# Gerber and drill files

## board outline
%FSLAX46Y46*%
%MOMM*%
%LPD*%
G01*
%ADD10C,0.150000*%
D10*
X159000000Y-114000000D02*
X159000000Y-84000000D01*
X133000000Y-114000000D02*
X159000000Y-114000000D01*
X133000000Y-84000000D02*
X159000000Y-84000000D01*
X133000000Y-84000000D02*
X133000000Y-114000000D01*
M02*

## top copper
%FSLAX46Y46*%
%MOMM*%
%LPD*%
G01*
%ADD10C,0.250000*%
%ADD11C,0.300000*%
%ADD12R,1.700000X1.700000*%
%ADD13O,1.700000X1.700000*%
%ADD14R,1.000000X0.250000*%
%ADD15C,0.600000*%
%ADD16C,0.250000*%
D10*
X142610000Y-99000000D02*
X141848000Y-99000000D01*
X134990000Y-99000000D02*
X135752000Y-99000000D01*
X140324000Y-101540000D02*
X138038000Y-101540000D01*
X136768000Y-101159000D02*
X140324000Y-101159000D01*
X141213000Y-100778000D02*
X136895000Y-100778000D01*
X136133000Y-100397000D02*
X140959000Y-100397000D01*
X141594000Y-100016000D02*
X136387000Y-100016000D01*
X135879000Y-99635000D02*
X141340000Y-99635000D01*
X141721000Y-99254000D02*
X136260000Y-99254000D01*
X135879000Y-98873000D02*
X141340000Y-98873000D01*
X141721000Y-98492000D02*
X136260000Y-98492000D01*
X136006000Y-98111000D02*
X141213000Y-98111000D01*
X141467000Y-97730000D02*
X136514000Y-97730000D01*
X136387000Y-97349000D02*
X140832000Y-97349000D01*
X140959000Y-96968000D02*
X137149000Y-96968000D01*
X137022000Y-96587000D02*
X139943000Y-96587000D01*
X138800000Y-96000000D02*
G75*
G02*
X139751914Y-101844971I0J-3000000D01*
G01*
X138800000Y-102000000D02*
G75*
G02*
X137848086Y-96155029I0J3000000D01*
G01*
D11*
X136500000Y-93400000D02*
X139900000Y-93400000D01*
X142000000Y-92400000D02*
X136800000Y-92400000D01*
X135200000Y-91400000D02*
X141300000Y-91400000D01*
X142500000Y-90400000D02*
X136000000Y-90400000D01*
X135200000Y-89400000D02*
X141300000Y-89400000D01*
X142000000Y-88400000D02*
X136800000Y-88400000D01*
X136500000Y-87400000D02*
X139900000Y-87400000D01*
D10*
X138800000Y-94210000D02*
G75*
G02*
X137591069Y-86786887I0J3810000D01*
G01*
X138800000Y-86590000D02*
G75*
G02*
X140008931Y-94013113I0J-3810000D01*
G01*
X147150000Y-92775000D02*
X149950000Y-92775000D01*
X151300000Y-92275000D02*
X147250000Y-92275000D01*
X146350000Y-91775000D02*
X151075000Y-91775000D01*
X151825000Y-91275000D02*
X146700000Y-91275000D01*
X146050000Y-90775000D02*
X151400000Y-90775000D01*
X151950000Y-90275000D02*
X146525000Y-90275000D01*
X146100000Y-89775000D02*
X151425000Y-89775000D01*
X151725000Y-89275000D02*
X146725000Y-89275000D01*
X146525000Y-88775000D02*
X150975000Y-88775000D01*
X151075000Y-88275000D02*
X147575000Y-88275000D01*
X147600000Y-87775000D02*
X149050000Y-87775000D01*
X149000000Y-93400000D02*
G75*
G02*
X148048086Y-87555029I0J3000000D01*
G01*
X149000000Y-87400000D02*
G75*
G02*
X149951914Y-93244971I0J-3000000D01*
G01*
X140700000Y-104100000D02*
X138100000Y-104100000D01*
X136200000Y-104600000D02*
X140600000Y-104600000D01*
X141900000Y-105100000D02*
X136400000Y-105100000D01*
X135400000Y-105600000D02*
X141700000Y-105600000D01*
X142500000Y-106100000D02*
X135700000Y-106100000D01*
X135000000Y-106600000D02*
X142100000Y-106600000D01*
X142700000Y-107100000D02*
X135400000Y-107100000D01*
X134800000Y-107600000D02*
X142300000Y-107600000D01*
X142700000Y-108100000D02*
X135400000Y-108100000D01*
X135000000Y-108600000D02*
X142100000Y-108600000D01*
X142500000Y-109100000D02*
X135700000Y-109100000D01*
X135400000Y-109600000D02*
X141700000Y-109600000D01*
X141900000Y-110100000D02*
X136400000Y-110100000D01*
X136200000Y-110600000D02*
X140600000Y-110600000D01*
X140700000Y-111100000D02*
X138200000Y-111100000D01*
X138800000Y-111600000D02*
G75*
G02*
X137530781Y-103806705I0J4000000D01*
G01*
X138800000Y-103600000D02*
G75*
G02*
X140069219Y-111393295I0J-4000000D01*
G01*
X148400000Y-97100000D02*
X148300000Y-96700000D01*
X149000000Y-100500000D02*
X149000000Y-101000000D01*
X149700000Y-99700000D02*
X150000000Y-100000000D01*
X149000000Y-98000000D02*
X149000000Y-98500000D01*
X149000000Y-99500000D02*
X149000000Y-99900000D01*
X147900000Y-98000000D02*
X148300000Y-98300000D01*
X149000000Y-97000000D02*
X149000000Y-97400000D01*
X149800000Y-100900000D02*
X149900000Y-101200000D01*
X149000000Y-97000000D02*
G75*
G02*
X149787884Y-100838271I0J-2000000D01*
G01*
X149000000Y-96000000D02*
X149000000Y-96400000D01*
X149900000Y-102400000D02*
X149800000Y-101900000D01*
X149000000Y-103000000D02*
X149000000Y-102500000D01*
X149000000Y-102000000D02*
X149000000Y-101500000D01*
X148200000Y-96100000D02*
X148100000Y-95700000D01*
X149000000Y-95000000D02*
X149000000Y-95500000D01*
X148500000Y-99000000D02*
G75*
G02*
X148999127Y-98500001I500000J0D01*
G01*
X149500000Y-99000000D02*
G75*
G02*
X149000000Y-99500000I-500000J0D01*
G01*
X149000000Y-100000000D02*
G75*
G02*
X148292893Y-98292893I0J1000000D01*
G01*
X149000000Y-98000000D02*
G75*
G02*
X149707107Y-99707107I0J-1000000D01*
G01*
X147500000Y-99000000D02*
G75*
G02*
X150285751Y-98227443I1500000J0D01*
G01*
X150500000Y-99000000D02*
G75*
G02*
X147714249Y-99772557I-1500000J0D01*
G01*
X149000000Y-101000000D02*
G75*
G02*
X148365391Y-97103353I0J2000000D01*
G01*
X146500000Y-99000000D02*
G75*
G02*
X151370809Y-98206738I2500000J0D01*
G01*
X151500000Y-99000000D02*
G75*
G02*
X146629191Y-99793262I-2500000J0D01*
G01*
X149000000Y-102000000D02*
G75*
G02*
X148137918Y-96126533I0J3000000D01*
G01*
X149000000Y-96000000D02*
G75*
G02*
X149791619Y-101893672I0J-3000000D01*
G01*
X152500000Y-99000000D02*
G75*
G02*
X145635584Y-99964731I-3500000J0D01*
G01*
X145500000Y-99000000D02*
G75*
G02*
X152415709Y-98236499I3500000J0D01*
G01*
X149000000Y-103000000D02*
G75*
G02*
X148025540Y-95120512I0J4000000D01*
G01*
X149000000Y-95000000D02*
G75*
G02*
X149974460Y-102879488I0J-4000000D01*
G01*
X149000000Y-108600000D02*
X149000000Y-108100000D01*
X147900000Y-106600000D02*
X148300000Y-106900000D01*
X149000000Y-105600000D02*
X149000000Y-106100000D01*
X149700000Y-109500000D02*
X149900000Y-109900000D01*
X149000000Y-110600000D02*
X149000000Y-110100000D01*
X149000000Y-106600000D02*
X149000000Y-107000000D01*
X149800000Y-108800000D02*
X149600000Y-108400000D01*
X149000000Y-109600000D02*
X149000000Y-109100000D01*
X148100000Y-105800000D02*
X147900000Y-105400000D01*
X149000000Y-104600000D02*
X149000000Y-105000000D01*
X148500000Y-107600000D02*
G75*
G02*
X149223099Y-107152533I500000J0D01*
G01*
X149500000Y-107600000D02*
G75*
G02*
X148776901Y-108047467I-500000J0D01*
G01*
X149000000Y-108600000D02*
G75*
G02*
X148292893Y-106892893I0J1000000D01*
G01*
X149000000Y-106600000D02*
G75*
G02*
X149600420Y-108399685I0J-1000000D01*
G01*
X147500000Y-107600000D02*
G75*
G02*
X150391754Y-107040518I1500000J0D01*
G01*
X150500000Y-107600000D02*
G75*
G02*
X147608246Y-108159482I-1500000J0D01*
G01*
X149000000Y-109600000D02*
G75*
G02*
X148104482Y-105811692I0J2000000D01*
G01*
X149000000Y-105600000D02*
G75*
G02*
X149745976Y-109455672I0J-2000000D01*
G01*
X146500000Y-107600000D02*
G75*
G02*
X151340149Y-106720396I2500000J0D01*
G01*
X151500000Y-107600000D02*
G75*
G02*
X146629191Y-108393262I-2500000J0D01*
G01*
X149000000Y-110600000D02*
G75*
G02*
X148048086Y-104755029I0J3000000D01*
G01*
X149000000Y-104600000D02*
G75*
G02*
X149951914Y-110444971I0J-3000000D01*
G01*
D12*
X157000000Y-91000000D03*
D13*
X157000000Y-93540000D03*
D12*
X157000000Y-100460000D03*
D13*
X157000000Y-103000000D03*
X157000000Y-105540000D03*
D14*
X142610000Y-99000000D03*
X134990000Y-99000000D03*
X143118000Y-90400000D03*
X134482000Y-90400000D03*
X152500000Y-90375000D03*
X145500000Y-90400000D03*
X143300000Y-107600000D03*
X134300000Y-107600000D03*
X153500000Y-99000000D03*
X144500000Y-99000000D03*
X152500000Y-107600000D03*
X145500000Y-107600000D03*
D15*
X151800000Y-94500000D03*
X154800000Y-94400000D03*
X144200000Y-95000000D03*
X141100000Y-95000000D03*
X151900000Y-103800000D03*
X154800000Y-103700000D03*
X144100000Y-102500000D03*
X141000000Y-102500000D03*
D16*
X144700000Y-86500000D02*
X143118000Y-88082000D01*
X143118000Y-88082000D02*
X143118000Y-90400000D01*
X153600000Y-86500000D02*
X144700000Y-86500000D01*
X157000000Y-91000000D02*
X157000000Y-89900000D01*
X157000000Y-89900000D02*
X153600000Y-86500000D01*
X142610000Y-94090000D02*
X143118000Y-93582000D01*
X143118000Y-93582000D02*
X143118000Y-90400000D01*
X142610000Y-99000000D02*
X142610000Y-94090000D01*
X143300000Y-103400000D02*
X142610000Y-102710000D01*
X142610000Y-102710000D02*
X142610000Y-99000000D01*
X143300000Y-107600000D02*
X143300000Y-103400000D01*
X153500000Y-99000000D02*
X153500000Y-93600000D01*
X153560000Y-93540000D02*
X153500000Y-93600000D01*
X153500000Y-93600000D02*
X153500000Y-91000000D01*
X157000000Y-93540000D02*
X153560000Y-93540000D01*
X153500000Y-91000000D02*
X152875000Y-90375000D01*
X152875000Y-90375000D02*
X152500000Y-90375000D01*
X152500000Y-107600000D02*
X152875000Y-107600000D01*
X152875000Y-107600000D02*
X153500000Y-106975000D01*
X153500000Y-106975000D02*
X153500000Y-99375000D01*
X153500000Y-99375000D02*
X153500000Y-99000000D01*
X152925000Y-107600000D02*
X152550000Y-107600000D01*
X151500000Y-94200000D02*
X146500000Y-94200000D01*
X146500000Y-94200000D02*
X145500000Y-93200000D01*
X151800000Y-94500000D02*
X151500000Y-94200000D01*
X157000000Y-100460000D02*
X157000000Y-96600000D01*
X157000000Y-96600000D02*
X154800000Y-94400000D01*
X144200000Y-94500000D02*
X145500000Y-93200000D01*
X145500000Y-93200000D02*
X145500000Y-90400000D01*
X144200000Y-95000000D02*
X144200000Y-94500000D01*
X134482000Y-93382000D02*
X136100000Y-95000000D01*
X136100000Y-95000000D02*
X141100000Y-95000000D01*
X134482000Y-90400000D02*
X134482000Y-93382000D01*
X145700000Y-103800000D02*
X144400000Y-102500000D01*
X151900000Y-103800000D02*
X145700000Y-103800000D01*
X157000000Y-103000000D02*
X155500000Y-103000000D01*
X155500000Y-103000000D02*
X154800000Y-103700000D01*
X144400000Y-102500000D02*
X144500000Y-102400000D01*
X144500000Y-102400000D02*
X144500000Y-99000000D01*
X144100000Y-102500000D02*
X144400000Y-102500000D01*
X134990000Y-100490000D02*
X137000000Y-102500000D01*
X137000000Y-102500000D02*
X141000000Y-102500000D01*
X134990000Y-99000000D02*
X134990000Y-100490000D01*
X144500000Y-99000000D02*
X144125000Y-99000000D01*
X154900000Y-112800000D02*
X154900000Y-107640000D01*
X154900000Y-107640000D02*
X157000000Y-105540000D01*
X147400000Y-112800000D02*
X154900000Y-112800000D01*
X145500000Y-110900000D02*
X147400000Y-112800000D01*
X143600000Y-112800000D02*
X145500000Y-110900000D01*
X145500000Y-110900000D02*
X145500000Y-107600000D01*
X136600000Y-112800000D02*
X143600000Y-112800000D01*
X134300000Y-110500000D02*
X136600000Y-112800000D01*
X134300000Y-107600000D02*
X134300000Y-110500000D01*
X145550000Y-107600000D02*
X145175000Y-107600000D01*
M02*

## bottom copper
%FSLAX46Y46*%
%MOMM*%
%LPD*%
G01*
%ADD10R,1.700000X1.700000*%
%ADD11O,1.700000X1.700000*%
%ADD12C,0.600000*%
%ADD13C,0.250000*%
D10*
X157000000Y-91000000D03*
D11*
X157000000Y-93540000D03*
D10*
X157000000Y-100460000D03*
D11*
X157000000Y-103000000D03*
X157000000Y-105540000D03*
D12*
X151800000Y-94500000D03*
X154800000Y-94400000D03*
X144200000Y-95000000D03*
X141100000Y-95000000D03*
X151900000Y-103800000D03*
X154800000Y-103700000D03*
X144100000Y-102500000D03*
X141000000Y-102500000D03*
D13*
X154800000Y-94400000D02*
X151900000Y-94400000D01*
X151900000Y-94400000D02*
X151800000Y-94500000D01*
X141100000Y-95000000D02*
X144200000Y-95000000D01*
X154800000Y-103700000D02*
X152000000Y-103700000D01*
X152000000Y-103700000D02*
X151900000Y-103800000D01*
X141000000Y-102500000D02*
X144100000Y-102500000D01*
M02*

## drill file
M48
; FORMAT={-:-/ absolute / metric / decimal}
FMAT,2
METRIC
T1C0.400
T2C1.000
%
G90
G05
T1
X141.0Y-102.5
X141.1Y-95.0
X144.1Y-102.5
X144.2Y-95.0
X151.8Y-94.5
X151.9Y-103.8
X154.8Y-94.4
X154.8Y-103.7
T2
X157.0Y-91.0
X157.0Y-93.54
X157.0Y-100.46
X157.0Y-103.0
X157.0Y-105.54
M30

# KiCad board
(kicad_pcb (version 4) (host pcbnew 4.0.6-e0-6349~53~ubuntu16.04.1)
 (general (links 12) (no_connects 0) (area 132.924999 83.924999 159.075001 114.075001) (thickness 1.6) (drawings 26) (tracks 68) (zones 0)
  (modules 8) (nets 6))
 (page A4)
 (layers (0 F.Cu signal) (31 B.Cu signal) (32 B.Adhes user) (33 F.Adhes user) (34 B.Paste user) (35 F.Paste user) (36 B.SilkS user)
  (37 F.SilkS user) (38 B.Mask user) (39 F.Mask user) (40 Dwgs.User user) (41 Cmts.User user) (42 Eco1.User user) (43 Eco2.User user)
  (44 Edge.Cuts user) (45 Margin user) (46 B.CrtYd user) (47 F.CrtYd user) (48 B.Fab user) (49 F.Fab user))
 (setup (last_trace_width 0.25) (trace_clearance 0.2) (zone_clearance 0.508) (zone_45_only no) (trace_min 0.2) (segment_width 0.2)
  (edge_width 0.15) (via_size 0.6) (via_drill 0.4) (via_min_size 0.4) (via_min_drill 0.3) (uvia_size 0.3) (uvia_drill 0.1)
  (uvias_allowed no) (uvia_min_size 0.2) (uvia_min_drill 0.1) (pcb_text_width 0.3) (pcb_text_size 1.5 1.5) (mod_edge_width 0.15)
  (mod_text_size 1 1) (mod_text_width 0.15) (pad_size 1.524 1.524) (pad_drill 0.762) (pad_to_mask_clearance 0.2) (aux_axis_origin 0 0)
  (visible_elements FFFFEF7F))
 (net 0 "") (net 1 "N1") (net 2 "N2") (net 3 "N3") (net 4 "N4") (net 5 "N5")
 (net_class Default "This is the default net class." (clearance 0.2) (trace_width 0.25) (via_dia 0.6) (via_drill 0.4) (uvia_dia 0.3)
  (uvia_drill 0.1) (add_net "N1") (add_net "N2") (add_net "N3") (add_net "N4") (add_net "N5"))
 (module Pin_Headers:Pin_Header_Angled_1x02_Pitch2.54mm (layer F.Cu) (at 157 91)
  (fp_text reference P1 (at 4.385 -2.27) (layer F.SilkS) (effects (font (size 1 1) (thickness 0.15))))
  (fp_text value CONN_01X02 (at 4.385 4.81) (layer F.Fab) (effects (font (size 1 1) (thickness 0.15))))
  (pad 1 thru_hole rect (at 0 0) (size 1.7 1.7) (drill 1) (layers *.Cu *.Mask) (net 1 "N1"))
  (pad 2 thru_hole oval (at 0 2.54) (size 1.7 1.7) (drill 1) (layers *.Cu *.Mask) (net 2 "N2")))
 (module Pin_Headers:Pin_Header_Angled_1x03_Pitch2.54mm (layer F.Cu) (at 157 100.46)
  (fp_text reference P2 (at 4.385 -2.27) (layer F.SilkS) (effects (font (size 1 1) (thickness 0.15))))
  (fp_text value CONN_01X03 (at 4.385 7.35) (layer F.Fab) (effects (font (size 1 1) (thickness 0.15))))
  (pad 1 thru_hole rect (at 0 0) (size 1.7 1.7) (drill 1) (layers *.Cu *.Mask) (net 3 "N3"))
  (pad 2 thru_hole oval (at 0 2.54) (size 1.7 1.7) (drill 1) (layers *.Cu *.Mask) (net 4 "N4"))
  (pad 3 thru_hole oval (at 0 5.08) (size 1.7 1.7) (drill 1) (layers *.Cu *.Mask) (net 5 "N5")))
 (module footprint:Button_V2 (layer F.Cu) (at 138.8 99)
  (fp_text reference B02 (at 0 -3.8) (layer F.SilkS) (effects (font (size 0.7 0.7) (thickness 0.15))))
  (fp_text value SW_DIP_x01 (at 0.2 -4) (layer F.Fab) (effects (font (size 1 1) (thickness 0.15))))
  (fp_line (start 3.81 0) (end 3.048 0) (layer F.Cu) (width 0.25))
  (fp_line (start -3.81 0) (end -3.048 0) (layer F.Cu) (width 0.25))
  (fp_line (start 1.524 2.54) (end -0.762 2.54) (layer F.Cu) (width 0.25))
  (fp_line (start -2.032 2.159) (end 1.524 2.159) (layer F.Cu) (width 0.25))
  (fp_line (start 2.413 1.778) (end -1.905 1.778) (layer F.Cu) (width 0.25))
  (fp_line (start -2.667 1.397) (end 2.159 1.397) (layer F.Cu) (width 0.25))
  (fp_line (start 2.794 1.016) (end -2.413 1.016) (layer F.Cu) (width 0.25))
  (fp_line (start -2.921 0.635) (end 2.54 0.635) (layer F.Cu) (width 0.25))
  (fp_line (start 2.921 0.254) (end -2.54 0.254) (layer F.Cu) (width 0.25))
  (fp_line (start -2.921 -0.127) (end 2.54 -0.127) (layer F.Cu) (width 0.25))
  (fp_line (start 2.921 -0.508) (end -2.54 -0.508) (layer F.Cu) (width 0.25))
  (fp_line (start -2.794 -0.889) (end 2.413 -0.889) (layer F.Cu) (width 0.25))
  (fp_line (start 2.667 -1.27) (end -2.286 -1.27) (layer F.Cu) (width 0.25))
  (fp_line (start -2.413 -1.651) (end 2.032 -1.651) (layer F.Cu) (width 0.25))
  (fp_line (start 2.159 -2.032) (end -1.651 -2.032) (layer F.Cu) (width 0.25))
  (fp_line (start -1.778 -2.413) (end 1.143 -2.413) (layer F.Cu) (width 0.25))
  (fp_arc (start 0 0) (end 0 -3) (angle 161.5) (layer F.Cu) (width 0.25))
  (fp_arc (start 0 0) (end 0 3) (angle 161.5) (layer F.Cu) (width 0.25))
  (pad 1 smd rect (at 3.81 0) (size 1 0.25) (layers F.Cu F.Paste F.Mask) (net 1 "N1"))
  (pad 2 smd rect (at -3.81 0) (size 1 0.25) (layers F.Cu F.Paste F.Mask) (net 4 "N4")))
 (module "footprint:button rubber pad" (layer F.Cu) (at 138.8 90.4)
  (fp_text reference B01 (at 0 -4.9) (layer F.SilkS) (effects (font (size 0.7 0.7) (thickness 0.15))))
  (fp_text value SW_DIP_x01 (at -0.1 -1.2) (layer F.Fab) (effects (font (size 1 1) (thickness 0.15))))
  (fp_line (start -2.3 3) (end 1.1 3) (layer F.Cu) (width 0.3)) (fp_line (start 3.2 2) (end -2 2) (layer F.Cu) (width 0.3))
  (fp_line (start -3.6 1) (end 2.5 1) (layer F.Cu) (width 0.3))
  (fp_line (start 3.7 0) (end -2.8 0) (layer F.Cu) (width 0.3))
  (fp_line (start -3.6 -1) (end 2.5 -1) (layer F.Cu) (width 0.3))
  (fp_line (start 3.2 -2) (end -2 -2) (layer F.Cu) (width 0.3))
  (fp_line (start -2.3 -3) (end 1.1 -3) (layer F.Cu) (width 0.3))
  (fp_arc (start 0 0) (end 0 3.81) (angle 161.5) (layer F.Cu) (width 0.25))
  (fp_arc (start 0 0) (end 0 -3.81) (angle 161.5) (layer F.Cu) (width 0.25))
  (pad 1 smd rect (at 4.318 0) (size 1 0.25) (layers F.Cu F.Paste F.Mask) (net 1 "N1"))
  (pad 2 smd rect (at -4.318 0) (size 1 0.25) (layers F.Cu F.Paste F.Mask) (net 3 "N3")))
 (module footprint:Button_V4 (layer F.Cu) (at 149 90.4)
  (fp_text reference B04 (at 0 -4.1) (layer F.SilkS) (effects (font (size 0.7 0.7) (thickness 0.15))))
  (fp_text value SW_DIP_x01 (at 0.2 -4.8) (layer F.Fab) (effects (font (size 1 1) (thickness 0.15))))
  (fp_line (start -1.85 2.375) (end 0.95 2.375) (layer F.Cu) (width 0.25))
  (fp_line (start 2.3 1.875) (end -1.75 1.875) (layer F.Cu) (width 0.25))
  (fp_line (start -2.65 1.375) (end 2.075 1.375) (layer F.Cu) (width 0.25))
  (fp_line (start 2.825 0.875) (end -2.3 0.875) (layer F.Cu) (width 0.25))
  (fp_line (start -2.95 0.375) (end 2.4 0.375) (layer F.Cu) (width 0.25))
  (fp_line (start 2.95 -0.125) (end -2.475 -0.125) (layer F.Cu) (width 0.25))
  (fp_line (start -2.9 -0.625) (end 2.425 -0.625) (layer F.Cu) (width 0.25))
  (fp_line (start 2.725 -1.125) (end -2.275 -1.125) (layer F.Cu) (width 0.25))
  (fp_line (start -2.475 -1.625) (end 1.975 -1.625) (layer F.Cu) (width 0.25))
  (fp_line (start 2.075 -2.125) (end -1.425 -2.125) (layer F.Cu) (width 0.25))
  (fp_line (start -1.4 -2.625) (end 0.05 -2.625) (layer F.Cu) (width 0.25))
  (fp_arc (start 0 0) (end 0 3) (angle 161.5) (layer F.Cu) (width 0.25))
  (fp_arc (start 0 0) (end 0 -3) (angle 161.5) (layer F.Cu) (width 0.25))
  (pad 1 smd rect (at 3.5 -0.025) (size 1 0.25) (layers F.Cu F.Paste F.Mask) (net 2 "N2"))
  (pad 2 smd rect (at -3.5 0) (size 1 0.25) (layers F.Cu F.Paste F.Mask) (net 3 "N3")))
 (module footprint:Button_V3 (layer F.Cu) (at 138.8 107.6)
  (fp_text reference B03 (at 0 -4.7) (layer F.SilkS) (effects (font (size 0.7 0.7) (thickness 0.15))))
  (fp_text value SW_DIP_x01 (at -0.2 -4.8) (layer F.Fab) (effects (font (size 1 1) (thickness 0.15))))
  (fp_line (start 1.9 -3.5) (end -0.7 -3.5) (layer F.Cu) (width 0.25))
  (fp_line (start -2.6 -3) (end 1.8 -3) (layer F.Cu) (width 0.25))
  (fp_line (start 3.1 -2.5) (end -2.4 -2.5) (layer F.Cu) (width 0.25))
  (fp_line (start -3.4 -2) (end 2.9 -2) (layer F.Cu) (width 0.25))
  (fp_line (start 3.7 -1.5) (end -3.1 -1.5) (layer F.Cu) (width 0.25))
  (fp_line (start -3.8 -1) (end 3.3 -1) (layer F.Cu) (width 0.25))
  (fp_line (start 3.9 -0.5) (end -3.4 -0.5) (layer F.Cu) (width 0.25)) (fp_line (start -4 0) (end 3.5 0) (layer F.Cu) (width 0.25))
  (fp_line (start 3.9 0.5) (end -3.4 0.5) (layer F.Cu) (width 0.25))
  (fp_line (start -3.8 1) (end 3.3 1) (layer F.Cu) (width 0.25))
  (fp_line (start 3.7 1.5) (end -3.1 1.5) (layer F.Cu) (width 0.25))
  (fp_line (start -3.4 2) (end 2.9 2) (layer F.Cu) (width 0.25))
  (fp_line (start 3.1 2.5) (end -2.4 2.5) (layer F.Cu) (width 0.25))
  (fp_line (start -2.6 3) (end 1.8 3) (layer F.Cu) (width 0.25))
  (fp_line (start 1.9 3.5) (end -0.6 3.5) (layer F.Cu) (width 0.25))
  (fp_arc (start 0 0) (end 0 4) (angle 161.5) (layer F.Cu) (width 0.25))
  (fp_arc (start 0 0) (end 0 -4) (angle 161.5) (layer F.Cu) (width 0.25))
  (pad 1 smd rect (at 4.5 0) (size 1 0.25) (layers F.Cu F.Paste F.Mask) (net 1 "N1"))
  (pad 2 smd rect (at -4.5 0) (size 1 0.25) (layers F.Cu F.Paste F.Mask) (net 5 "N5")))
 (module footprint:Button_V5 (layer F.Cu) (at 149 99)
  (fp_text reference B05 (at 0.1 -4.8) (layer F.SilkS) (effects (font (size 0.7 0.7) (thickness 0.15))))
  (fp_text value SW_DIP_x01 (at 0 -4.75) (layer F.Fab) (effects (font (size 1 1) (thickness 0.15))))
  (fp_line (start -0.6 -1.9) (end -0.7 -2.3) (layer F.Cu) (width 0.25)) (fp_line (start 0 1.5) (end 0 2) (layer F.Cu) (width 0.25))
  (fp_line (start 0.7 0.7) (end 1 1) (layer F.Cu) (width 0.25))
  (fp_line (start 0 -1) (end 0 -0.5) (layer F.Cu) (width 0.25))
  (fp_line (start 0 0.5) (end 0 0.9) (layer F.Cu) (width 0.25))
  (fp_line (start -1.1 -1) (end -0.7 -0.7) (layer F.Cu) (width 0.25))
  (fp_line (start 0 -2) (end 0 -1.6) (layer F.Cu) (width 0.25))
  (fp_line (start 0.8 1.9) (end 0.9 2.2) (layer F.Cu) (width 0.25))
  (fp_arc (start 0 0) (end 0 -2) (angle 156.8) (layer F.Cu) (width 0.25))
  (fp_line (start 0 -3) (end 0 -2.6) (layer F.Cu) (width 0.25))
  (fp_line (start 0.9 3.4) (end 0.8 2.9) (layer F.Cu) (width 0.25)) (fp_line (start 0 4) (end 0 3.5) (layer F.Cu) (width 0.25))
  (fp_line (start 0 3) (end 0 2.5) (layer F.Cu) (width 0.25))
  (fp_line (start -0.8 -2.9) (end -0.9 -3.3) (layer F.Cu) (width 0.25))
  (fp_line (start 0 -4) (end 0 -3.5) (layer F.Cu) (width 0.25))
  (fp_arc (start 0 0) (end -0.5 0) (angle 89.9) (layer F.Cu) (width 0.25))
  (fp_arc (start 0 0) (end 0.5 0) (angle 90) (layer F.Cu) (width 0.25))
  (fp_arc (start 0 0) (end 0 1) (angle 135) (layer F.Cu) (width 0.25))
  (fp_arc (start 0 0) (end 0 -1) (angle 135) (layer F.Cu) (width 0.25))
  (fp_arc (start 0 0) (end -1.5 0) (angle 149) (layer F.Cu) (width 0.25))
  (fp_arc (start 0 0) (end 1.5 0) (angle 149) (layer F.Cu) (width 0.25))
  (fp_arc (start 0 0) (end 0 2) (angle 161.5) (layer F.Cu) (width 0.25))
  (fp_arc (start 0 0) (end -2.5 0) (angle 161.5) (layer F.Cu) (width 0.25))
  (fp_arc (start 0 0) (end 2.5 0) (angle 161.5) (layer F.Cu) (width 0.25))
  (fp_arc (start 0 0) (end 0 3) (angle 163.3) (layer F.Cu) (width 0.25))
  (fp_arc (start 0 0) (end 0 -3) (angle 164.7) (layer F.Cu) (width 0.25))
  (fp_arc (start 0 0) (end 3.5 0) (angle 164) (layer F.Cu) (width 0.25))
  (fp_arc (start 0 0) (end -3.5 0) (angle 167.4) (layer F.Cu) (width 0.25))
  (fp_arc (start 0 0) (end 0 4) (angle 165.9) (layer F.Cu) (width 0.25))
  (fp_arc (start 0 0) (end 0 -4) (angle 165.9) (layer F.Cu) (width 0.25))
  (pad 1 smd rect (at 4.5 0) (size 1 0.25) (layers F.Cu F.Paste F.Mask) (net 2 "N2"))
  (pad 2 smd rect (at -4.5 0) (size 1 0.25) (layers F.Cu F.Paste F.Mask) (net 4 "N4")))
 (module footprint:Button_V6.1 (layer F.Cu) (at 149 107.6)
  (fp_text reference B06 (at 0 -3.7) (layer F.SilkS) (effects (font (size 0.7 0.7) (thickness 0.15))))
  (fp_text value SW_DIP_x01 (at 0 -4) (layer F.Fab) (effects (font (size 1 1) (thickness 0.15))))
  (fp_line (start 0 1) (end 0 0.5) (layer F.Cu) (width 0.25))
  (fp_line (start -1.1 -1) (end -0.7 -0.7) (layer F.Cu) (width 0.25))
  (fp_line (start 0 -2) (end 0 -1.5) (layer F.Cu) (width 0.25))
  (fp_line (start 0.7 1.9) (end 0.9 2.3) (layer F.Cu) (width 0.25)) (fp_line (start 0 3) (end 0 2.5) (layer F.Cu) (width 0.25))
  (fp_line (start 0 -1) (end 0 -0.6) (layer F.Cu) (width 0.25))
  (fp_line (start 0.8 1.2) (end 0.6 0.8) (layer F.Cu) (width 0.25)) (fp_line (start 0 2) (end 0 1.5) (layer F.Cu) (width 0.25))
  (fp_line (start -0.9 -1.8) (end -1.1 -2.2) (layer F.Cu) (width 0.25))
  (fp_line (start 0 -3) (end 0 -2.6) (layer F.Cu) (width 0.25))
  (fp_arc (start 0 0) (end -0.5 0) (angle 116.5) (layer F.Cu) (width 0.25))
  (fp_arc (start 0 0) (end 0.5 0) (angle 116.5) (layer F.Cu) (width 0.25))
  (fp_arc (start 0 0) (end 0 1) (angle 135) (layer F.Cu) (width 0.25))
  (fp_arc (start 0 0) (end 0 -1) (angle 143.1) (layer F.Cu) (width 0.25))
  (fp_arc (start 0 0) (end -1.5 0) (angle 158.1) (layer F.Cu) (width 0.25))
  (fp_arc (start 0 0) (end 1.5 0) (angle 158.1) (layer F.Cu) (width 0.25))
  (fp_arc (start 0 0) (end 0 2) (angle 153.4) (layer F.Cu) (width 0.25))
  (fp_arc (start 0 0) (end 0 -2) (angle 158.1) (layer F.Cu) (width 0.25))
  (fp_arc (start 0 0) (end -2.5 0) (angle 159.4) (layer F.Cu) (width 0.25))
  (fp_arc (start 0 0) (end 2.5 0) (angle 161.5) (layer F.Cu) (width 0.25))
  (fp_arc (start 0 0) (end 0 3) (angle 161.5) (layer F.Cu) (width 0.25))
  (fp_arc (start 0 0) (end 0 -3) (angle 161.5) (layer F.Cu) (width 0.25))
  (pad 1 smd rect (at 3.5 0) (size 1 0.25) (layers F.Cu F.Paste F.Mask) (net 2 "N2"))
  (pad 2 smd rect (at -3.5 0) (size 1 0.25) (layers F.Cu F.Paste F.Mask) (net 5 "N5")))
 (gr_line (start 159 114) (end 159 84) (layer Edge.Cuts) (width 0.15))
 (gr_line (start 133 114) (end 159 114) (layer Edge.Cuts) (width 0.15))
 (gr_line (start 133 84) (end 159 84) (layer Edge.Cuts) (width 0.15))
 (gr_line (start 133 84) (end 133 114) (layer Edge.Cuts) (width 0.15))
 (segment (start 144.7 86.5) (end 143.118 88.082) (width 0.25) (layer F.Cu) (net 1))
 (segment (start 143.118 88.082) (end 143.118 90.4) (width 0.25) (layer F.Cu) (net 1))
 (segment (start 153.6 86.5) (end 144.7 86.5) (width 0.25) (layer F.Cu) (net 1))
 (segment (start 157 91) (end 157 89.9) (width 0.25) (layer F.Cu) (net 1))
 (segment (start 157 89.9) (end 153.6 86.5) (width 0.25) (layer F.Cu) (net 1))
 (segment (start 142.61 94.09) (end 143.118 93.582) (width 0.25) (layer F.Cu) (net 1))
 (segment (start 143.118 93.582) (end 143.118 90.4) (width 0.25) (layer F.Cu) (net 1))
 (segment (start 142.61 99) (end 142.61 94.09) (width 0.25) (layer F.Cu) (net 1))
 (segment (start 143.3 103.4) (end 142.61 102.71) (width 0.25) (layer F.Cu) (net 1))
 (segment (start 142.61 102.71) (end 142.61 99) (width 0.25) (layer F.Cu) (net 1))
 (segment (start 143.3 107.6) (end 143.3 103.4) (width 0.25) (layer F.Cu) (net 1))
 (segment (start 153.5 99) (end 153.5 93.6) (width 0.25) (layer F.Cu) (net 2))
 (segment (start 153.56 93.54) (end 153.5 93.6) (width 0.25) (layer F.Cu) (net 2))
 (segment (start 153.5 93.6) (end 153.5 91) (width 0.25) (layer F.Cu) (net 2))
 (segment (start 157 93.54) (end 153.56 93.54) (width 0.25) (layer F.Cu) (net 2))
 (segment (start 153.5 91) (end 152.875 90.375) (width 0.25) (layer F.Cu) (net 2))
 (segment (start 152.875 90.375) (end 152.5 90.375) (width 0.25) (layer F.Cu) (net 2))
 (segment (start 152.5 107.6) (end 152.875 107.6) (width 0.25) (layer F.Cu) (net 2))
 (segment (start 152.875 107.6) (end 153.5 106.975) (width 0.25) (layer F.Cu) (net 2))
 (segment (start 153.5 106.975) (end 153.5 99.375) (width 0.25) (layer F.Cu) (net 2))
 (segment (start 153.5 99.375) (end 153.5 99) (width 0.25) (layer F.Cu) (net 2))
 (segment (start 152.925 107.6) (end 152.55 107.6) (width 0.25) (layer F.Cu) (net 2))
 (segment (start 151.5 94.2) (end 146.5 94.2) (width 0.25) (layer F.Cu) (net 3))
 (segment (start 146.5 94.2) (end 145.5 93.2) (width 0.25) (layer F.Cu) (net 3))
 (segment (start 151.8 94.5) (end 151.5 94.2) (width 0.25) (layer F.Cu) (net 3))
 (segment (start 154.8 94.4) (end 151.9 94.4) (width 0.25) (layer B.Cu) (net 3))
 (segment (start 151.9 94.4) (end 151.8 94.5) (width 0.25) (layer B.Cu) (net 3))
 (via (at 151.8 94.5) (size 0.6) (drill 0.4) (layers F.Cu B.Cu) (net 3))
 (segment (start 157 100.46) (end 157 96.6) (width 0.25) (layer F.Cu) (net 3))
 (segment (start 157 96.6) (end 154.8 94.4) (width 0.25) (layer F.Cu) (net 3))
 (via (at 154.8 94.4) (size 0.6) (drill 0.4) (layers F.Cu B.Cu) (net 3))
 (segment (start 144.2 94.5) (end 145.5 93.2) (width 0.25) (layer F.Cu) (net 3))
 (segment (start 145.5 93.2) (end 145.5 90.4) (width 0.25) (layer F.Cu) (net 3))
 (segment (start 144.2 95) (end 144.2 94.5) (width 0.25) (layer F.Cu) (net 3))
 (segment (start 141.1 95) (end 144.2 95) (width 0.25) (layer B.Cu) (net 3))
 (via (at 144.2 95) (size 0.6) (drill 0.4) (layers F.Cu B.Cu) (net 3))
 (segment (start 134.482 93.382) (end 136.1 95) (width 0.25) (layer F.Cu) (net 3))
 (segment (start 136.1 95) (end 141.1 95) (width 0.25) (layer F.Cu) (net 3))
 (via (at 141.1 95) (size 0.6) (drill 0.4) (layers F.Cu B.Cu) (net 3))
 (segment (start 134.482 90.4) (end 134.482 93.382) (width 0.25) (layer F.Cu) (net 3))
 (segment (start 145.7 103.8) (end 144.4 102.5) (width 0.25) (layer F.Cu) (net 4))
 (segment (start 151.9 103.8) (end 145.7 103.8) (width 0.25) (layer F.Cu) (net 4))
 (segment (start 154.8 103.7) (end 152 103.7) (width 0.25) (layer B.Cu) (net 4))
 (segment (start 152 103.7) (end 151.9 103.8) (width 0.25) (layer B.Cu) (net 4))
 (via (at 151.9 103.8) (size 0.6) (drill 0.4) (layers F.Cu B.Cu) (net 4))
 (segment (start 157 103) (end 155.5 103) (width 0.25) (layer F.Cu) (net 4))
 (segment (start 155.5 103) (end 154.8 103.7) (width 0.25) (layer F.Cu) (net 4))
 (via (at 154.8 103.7) (size 0.6) (drill 0.4) (layers F.Cu B.Cu) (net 4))
 (segment (start 144.4 102.5) (end 144.5 102.4) (width 0.25) (layer F.Cu) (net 4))
 (segment (start 144.5 102.4) (end 144.5 99) (width 0.25) (layer F.Cu) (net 4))
 (segment (start 144.1 102.5) (end 144.4 102.5) (width 0.25) (layer F.Cu) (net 4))
 (segment (start 141 102.5) (end 144.1 102.5) (width 0.25) (layer B.Cu) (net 4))
 (via (at 144.1 102.5) (size 0.6) (drill 0.4) (layers F.Cu B.Cu) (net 4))
 (segment (start 134.99 100.49) (end 137 102.5) (width 0.25) (layer F.Cu) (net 4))
 (segment (start 137 102.5) (end 141 102.5) (width 0.25) (layer F.Cu) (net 4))
 (via (at 141 102.5) (size 0.6) (drill 0.4) (layers F.Cu B.Cu) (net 4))
 (segment (start 134.99 99) (end 134.99 100.49) (width 0.25) (layer F.Cu) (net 4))
 (segment (start 144.5 99) (end 144.125 99) (width 0.25) (layer F.Cu) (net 4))
 (segment (start 154.9 112.8) (end 154.9 107.64) (width 0.25) (layer F.Cu) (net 5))
 (segment (start 154.9 107.64) (end 157 105.54) (width 0.25) (layer F.Cu) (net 5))
 (segment (start 147.4 112.8) (end 154.9 112.8) (width 0.25) (layer F.Cu) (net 5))
 (segment (start 145.5 110.9) (end 147.4 112.8) (width 0.25) (layer F.Cu) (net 5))
 (segment (start 143.6 112.8) (end 145.5 110.9) (width 0.25) (layer F.Cu) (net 5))
 (segment (start 145.5 110.9) (end 145.5 107.6) (width 0.25) (layer F.Cu) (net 5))
 (segment (start 136.6 112.8) (end 143.6 112.8) (width 0.25) (layer F.Cu) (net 5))
 (segment (start 134.3 110.5) (end 136.6 112.8) (width 0.25) (layer F.Cu) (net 5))
 (segment (start 134.3 107.6) (end 134.3 110.5) (width 0.25) (layer F.Cu) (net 5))
 (segment (start 145.55 107.6) (end 145.175 107.6) (width 0.25) (layer F.Cu) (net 5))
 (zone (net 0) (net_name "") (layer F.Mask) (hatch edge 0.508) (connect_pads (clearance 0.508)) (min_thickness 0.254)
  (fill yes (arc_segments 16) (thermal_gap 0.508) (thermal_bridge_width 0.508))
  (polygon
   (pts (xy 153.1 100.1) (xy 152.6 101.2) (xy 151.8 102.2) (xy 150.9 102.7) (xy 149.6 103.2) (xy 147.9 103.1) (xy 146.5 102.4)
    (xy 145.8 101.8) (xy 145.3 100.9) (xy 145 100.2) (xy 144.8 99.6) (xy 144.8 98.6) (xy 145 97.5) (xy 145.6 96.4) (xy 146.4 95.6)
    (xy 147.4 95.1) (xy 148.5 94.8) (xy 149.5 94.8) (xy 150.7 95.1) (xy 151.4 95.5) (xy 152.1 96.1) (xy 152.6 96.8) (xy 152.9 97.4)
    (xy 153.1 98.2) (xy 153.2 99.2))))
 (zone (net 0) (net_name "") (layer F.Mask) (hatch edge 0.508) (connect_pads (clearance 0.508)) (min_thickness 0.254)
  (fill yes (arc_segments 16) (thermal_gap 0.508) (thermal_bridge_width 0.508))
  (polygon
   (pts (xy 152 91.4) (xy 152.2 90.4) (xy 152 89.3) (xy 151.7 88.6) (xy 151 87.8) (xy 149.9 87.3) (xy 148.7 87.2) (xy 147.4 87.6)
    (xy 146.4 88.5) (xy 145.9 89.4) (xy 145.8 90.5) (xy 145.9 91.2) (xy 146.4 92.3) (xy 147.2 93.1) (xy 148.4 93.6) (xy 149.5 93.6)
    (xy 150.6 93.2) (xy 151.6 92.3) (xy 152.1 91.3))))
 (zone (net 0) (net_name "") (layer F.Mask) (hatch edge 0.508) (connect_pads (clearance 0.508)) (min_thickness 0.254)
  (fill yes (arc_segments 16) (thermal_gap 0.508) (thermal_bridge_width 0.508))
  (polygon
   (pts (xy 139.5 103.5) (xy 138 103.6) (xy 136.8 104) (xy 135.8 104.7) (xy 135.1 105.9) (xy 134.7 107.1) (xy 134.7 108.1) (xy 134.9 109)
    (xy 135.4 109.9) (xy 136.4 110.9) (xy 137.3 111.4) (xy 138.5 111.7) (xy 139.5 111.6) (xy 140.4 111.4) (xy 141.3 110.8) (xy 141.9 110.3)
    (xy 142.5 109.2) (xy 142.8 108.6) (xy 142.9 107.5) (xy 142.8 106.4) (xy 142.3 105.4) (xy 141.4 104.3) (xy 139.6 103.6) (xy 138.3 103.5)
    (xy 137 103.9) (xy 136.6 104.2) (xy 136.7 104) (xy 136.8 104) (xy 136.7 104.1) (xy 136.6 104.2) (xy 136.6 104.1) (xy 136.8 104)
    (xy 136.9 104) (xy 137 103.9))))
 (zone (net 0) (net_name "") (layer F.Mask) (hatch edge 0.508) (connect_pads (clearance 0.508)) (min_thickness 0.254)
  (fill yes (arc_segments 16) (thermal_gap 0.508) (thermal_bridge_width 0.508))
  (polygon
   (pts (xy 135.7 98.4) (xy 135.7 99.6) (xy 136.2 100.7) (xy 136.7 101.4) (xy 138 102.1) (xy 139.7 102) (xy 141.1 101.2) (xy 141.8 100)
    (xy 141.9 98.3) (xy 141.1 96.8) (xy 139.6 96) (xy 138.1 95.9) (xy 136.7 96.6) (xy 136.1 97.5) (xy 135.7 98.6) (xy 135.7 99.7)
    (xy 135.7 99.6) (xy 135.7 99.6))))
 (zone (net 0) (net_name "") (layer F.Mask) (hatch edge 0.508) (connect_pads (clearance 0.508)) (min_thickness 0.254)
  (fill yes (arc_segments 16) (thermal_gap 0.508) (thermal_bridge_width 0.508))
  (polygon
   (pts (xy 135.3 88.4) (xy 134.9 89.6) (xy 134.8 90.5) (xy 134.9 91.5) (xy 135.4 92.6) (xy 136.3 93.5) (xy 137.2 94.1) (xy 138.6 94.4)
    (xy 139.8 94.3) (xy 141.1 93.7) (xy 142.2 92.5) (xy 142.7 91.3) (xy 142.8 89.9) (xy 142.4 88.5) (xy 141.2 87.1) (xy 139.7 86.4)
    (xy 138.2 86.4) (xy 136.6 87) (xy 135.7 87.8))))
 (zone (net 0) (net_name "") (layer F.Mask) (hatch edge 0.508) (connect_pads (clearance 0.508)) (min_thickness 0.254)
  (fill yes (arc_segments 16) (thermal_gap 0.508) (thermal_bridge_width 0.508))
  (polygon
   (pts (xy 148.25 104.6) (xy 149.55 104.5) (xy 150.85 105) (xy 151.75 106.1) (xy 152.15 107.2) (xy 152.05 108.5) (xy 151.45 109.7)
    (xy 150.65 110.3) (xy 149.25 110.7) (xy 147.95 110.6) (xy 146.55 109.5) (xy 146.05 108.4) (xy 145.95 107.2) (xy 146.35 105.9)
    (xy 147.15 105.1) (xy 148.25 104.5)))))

